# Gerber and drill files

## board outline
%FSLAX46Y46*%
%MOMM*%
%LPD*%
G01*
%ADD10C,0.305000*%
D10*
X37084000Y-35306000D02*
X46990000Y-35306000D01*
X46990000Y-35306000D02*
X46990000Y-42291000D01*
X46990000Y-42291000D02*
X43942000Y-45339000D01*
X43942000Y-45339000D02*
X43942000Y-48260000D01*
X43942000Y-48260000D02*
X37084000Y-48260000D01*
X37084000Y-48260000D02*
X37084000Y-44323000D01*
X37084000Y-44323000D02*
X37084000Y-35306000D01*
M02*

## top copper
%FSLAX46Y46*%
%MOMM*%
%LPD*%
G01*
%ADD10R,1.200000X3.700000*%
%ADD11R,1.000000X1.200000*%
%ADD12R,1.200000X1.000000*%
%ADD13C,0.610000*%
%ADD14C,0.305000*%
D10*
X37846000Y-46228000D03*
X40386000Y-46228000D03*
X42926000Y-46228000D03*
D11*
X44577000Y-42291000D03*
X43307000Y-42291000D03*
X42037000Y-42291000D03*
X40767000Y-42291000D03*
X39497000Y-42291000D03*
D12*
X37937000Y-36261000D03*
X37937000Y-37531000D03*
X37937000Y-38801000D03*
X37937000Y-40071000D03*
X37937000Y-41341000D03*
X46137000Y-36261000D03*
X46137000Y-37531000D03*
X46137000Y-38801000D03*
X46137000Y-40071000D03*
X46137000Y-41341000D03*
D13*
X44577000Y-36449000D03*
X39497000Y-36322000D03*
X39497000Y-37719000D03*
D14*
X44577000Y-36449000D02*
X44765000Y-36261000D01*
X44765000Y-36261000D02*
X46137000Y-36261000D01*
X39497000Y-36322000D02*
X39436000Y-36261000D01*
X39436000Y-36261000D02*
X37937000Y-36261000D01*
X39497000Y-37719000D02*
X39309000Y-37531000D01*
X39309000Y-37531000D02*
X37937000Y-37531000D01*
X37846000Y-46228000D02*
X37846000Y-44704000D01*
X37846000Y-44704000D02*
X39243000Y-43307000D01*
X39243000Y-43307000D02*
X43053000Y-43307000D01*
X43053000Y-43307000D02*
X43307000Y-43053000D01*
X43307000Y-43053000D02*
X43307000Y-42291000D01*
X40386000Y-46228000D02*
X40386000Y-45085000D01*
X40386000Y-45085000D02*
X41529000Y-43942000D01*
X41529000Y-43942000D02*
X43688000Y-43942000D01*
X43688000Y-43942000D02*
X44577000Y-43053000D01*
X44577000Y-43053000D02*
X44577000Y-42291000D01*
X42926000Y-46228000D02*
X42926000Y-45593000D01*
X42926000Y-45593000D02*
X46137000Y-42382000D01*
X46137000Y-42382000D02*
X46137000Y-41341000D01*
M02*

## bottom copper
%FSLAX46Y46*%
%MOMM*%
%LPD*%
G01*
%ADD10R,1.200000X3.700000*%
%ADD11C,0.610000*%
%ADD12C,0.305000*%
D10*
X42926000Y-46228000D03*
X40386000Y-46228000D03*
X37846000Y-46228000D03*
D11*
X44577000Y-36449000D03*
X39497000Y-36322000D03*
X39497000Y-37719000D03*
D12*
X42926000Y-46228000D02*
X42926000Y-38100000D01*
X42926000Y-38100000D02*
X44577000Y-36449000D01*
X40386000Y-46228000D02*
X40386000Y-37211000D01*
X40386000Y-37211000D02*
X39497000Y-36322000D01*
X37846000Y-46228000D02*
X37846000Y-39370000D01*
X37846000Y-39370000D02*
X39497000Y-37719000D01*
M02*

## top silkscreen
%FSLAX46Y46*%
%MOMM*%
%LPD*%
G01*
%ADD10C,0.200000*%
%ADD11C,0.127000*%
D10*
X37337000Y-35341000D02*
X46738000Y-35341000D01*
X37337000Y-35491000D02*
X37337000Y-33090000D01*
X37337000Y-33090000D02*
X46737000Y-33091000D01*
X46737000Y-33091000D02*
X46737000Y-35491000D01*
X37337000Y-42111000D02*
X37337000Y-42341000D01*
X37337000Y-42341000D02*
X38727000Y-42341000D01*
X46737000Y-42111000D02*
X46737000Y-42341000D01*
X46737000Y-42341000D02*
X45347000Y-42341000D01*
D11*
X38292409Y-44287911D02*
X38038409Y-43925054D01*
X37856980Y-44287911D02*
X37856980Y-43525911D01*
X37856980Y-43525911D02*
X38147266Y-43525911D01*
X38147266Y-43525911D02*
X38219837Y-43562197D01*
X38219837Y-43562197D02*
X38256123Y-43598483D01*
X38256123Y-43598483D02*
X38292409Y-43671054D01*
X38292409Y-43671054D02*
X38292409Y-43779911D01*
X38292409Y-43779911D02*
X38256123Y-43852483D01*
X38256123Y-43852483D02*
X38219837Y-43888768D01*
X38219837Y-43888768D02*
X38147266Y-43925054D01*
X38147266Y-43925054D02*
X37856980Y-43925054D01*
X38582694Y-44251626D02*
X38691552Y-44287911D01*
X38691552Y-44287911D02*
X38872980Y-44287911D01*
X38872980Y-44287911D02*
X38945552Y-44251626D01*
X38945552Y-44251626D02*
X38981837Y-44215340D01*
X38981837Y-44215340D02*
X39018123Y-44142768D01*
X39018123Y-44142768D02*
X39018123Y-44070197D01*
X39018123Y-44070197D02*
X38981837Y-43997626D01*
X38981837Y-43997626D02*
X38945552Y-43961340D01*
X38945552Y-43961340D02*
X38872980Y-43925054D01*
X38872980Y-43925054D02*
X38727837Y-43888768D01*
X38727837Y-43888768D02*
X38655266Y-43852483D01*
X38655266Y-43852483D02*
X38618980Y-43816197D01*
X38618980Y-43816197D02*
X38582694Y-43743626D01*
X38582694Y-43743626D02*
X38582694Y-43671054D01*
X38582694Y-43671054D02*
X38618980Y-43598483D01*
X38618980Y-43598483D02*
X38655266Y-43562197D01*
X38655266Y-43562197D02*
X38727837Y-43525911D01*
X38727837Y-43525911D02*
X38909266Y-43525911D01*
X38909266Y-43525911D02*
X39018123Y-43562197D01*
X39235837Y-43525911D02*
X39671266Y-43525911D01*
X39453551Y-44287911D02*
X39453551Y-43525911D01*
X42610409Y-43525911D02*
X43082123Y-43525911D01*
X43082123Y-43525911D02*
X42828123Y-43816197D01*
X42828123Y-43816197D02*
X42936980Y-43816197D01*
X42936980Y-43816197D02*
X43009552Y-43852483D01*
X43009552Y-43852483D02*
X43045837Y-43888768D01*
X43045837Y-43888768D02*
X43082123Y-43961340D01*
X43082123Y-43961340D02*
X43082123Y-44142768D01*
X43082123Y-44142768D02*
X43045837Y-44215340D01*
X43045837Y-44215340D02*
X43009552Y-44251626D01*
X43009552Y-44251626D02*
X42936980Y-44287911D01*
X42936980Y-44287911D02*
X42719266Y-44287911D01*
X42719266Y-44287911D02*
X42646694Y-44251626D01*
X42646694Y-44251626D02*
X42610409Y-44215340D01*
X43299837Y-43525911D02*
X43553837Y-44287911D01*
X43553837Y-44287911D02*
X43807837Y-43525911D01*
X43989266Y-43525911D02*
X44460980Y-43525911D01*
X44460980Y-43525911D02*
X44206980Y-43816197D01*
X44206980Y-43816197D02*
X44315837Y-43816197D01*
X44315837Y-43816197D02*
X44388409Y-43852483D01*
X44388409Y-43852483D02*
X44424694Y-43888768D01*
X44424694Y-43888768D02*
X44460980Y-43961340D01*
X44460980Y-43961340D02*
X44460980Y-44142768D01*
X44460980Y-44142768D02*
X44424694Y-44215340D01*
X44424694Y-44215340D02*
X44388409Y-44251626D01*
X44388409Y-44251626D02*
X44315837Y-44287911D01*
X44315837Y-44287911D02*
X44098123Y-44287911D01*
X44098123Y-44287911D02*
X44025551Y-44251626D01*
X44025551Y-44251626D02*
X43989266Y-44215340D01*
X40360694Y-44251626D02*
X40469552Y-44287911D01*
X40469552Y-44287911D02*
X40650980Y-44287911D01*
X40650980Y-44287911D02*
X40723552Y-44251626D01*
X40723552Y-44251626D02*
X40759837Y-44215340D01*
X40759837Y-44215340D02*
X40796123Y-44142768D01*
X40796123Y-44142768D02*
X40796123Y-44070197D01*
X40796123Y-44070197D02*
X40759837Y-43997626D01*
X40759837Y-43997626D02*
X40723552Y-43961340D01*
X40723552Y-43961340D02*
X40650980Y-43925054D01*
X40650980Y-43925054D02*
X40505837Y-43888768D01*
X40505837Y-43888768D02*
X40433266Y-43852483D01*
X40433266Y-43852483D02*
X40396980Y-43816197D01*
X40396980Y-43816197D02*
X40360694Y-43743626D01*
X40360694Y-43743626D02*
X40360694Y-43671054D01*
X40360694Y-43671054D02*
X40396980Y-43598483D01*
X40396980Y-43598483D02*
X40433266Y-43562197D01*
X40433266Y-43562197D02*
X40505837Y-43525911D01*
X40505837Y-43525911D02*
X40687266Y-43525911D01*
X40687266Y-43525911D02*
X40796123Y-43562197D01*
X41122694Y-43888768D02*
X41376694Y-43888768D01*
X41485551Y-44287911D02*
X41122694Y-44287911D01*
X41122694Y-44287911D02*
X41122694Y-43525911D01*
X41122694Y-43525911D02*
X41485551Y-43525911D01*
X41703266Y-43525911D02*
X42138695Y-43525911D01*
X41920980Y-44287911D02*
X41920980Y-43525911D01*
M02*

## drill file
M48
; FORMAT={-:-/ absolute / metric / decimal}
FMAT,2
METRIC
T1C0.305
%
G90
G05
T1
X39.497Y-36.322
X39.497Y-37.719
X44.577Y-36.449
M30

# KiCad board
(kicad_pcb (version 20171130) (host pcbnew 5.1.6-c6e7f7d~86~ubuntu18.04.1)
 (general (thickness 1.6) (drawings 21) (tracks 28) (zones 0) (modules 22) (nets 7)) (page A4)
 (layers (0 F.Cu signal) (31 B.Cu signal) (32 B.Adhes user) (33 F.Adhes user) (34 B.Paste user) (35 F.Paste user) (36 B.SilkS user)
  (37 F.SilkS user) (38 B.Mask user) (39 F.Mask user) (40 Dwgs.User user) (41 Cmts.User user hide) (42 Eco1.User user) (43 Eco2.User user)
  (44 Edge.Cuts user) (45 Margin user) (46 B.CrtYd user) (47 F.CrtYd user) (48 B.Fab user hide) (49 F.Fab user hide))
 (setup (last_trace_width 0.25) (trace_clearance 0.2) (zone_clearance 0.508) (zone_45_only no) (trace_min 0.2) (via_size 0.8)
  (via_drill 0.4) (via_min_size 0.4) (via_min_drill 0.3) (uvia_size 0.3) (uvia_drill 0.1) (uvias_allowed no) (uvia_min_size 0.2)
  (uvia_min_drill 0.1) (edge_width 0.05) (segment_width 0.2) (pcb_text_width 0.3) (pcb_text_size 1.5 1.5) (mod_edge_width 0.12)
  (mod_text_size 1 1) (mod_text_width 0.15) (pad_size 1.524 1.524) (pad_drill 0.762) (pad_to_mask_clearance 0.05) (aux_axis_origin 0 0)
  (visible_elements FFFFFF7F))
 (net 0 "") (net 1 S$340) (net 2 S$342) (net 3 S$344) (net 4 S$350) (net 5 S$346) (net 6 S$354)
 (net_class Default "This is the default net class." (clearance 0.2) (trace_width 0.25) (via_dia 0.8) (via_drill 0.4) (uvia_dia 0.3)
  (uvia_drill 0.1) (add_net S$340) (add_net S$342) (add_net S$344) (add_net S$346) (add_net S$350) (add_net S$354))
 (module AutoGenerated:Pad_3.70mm (layer F.Cu) (at 37.846 46.228)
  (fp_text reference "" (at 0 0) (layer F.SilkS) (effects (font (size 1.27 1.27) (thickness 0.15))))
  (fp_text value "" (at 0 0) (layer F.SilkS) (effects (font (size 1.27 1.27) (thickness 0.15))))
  (pad 1 smd rect (at 0 0 90) (size 3.7 1.2) (layers F.Cu F.Paste F.Mask) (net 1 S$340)))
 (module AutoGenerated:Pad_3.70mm (layer F.Cu) (at 40.386 46.228)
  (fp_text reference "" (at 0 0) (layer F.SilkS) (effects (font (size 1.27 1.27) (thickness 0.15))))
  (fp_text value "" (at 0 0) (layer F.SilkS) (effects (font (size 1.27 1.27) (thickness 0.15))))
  (pad 1 smd rect (at 0 0 90) (size 3.7 1.2) (layers F.Cu F.Paste F.Mask) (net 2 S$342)))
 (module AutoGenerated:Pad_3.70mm (layer F.Cu) (at 42.926 46.228)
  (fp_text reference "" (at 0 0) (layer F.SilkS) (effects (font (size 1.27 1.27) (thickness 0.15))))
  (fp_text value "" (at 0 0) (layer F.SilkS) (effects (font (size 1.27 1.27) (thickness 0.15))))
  (pad 1 smd rect (at 0 0 90) (size 3.7 1.2) (layers F.Cu F.Paste F.Mask) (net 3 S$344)))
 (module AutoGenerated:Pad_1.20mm (layer F.Cu) (at 44.577 42.291)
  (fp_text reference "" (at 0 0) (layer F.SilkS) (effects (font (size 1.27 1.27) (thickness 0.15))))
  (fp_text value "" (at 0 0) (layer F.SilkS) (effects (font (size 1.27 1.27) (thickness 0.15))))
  (pad 15 smd rect (at 0 0 270) (size 1.2 1) (layers F.Cu F.Paste F.Mask) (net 2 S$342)))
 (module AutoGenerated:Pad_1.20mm (layer F.Cu) (at 43.307 42.291)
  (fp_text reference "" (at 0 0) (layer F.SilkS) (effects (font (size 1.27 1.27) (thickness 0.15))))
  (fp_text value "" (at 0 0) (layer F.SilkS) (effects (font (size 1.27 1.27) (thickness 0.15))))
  (pad 14 smd rect (at 0 0 270) (size 1.2 1) (layers F.Cu F.Paste F.Mask) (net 1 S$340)))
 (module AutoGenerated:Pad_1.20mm (layer F.Cu) (at 42.037 42.291)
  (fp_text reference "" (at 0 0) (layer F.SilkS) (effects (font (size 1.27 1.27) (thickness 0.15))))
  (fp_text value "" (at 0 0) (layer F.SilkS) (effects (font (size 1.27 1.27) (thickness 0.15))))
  (pad 13 smd rect (at 0 0 270) (size 1.2 1) (layers F.Cu F.Paste F.Mask)))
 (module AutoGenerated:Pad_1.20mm (layer F.Cu) (at 40.767 42.291)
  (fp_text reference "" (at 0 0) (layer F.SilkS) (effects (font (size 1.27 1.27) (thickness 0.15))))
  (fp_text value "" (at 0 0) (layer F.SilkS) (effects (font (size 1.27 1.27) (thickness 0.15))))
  (pad 12 smd rect (at 0 0 270) (size 1.2 1) (layers F.Cu F.Paste F.Mask)))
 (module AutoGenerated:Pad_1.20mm (layer F.Cu) (at 39.497 42.291)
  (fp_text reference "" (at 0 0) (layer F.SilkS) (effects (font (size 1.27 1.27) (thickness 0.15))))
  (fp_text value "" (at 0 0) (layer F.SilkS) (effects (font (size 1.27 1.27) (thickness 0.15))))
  (pad 11 smd rect (at 0 0 270) (size 1.2 1) (layers F.Cu F.Paste F.Mask)))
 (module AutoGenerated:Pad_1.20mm (layer F.Cu) (at 37.937 36.261)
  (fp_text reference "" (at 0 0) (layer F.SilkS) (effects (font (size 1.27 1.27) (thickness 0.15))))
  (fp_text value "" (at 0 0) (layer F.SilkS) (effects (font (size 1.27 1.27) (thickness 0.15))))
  (pad 1 smd rect (at 0 0) (size 1.2 1) (layers F.Cu F.Paste F.Mask) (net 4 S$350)))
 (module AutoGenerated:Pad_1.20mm (layer F.Cu) (at 37.937 37.531)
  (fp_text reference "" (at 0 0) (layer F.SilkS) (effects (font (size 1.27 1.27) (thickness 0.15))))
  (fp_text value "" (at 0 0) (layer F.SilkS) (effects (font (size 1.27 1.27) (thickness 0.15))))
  (pad 2 smd rect (at 0 0) (size 1.2 1) (layers F.Cu F.Paste F.Mask) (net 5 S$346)))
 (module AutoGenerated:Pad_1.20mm (layer F.Cu) (at 37.937 38.801)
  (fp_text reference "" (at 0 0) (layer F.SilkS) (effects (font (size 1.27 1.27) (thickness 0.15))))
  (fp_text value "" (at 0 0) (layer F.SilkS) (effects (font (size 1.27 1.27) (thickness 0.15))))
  (pad 3 smd rect (at 0 0) (size 1.2 1) (layers F.Cu F.Paste F.Mask)))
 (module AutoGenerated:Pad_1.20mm (layer F.Cu) (at 37.937 40.071)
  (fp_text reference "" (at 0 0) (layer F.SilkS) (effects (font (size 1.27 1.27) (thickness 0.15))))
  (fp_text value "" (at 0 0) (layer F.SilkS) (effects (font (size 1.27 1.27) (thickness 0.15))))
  (pad 4 smd rect (at 0 0) (size 1.2 1) (layers F.Cu F.Paste F.Mask)))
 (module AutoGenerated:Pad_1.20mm (layer F.Cu) (at 37.937 41.341)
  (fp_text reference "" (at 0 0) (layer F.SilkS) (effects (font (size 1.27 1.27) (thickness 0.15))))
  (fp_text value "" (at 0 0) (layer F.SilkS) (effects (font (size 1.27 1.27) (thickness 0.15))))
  (pad 5 smd rect (at 0 0) (size 1.2 1) (layers F.Cu F.Paste F.Mask)))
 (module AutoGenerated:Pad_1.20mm (layer F.Cu) (at 46.137 36.261)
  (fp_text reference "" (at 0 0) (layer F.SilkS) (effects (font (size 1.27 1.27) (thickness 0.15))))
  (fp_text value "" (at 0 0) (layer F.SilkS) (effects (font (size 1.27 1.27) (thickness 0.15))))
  (pad 6 smd rect (at 0 0) (size 1.2 1) (layers F.Cu F.Paste F.Mask) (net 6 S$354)))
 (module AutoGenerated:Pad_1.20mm (layer F.Cu) (at 46.137 37.531)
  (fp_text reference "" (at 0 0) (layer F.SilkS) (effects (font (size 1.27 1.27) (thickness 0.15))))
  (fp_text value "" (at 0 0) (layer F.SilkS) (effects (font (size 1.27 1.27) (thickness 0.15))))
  (pad 7 smd rect (at 0 0) (size 1.2 1) (layers F.Cu F.Paste F.Mask)))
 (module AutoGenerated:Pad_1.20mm (layer F.Cu) (at 46.137 38.801)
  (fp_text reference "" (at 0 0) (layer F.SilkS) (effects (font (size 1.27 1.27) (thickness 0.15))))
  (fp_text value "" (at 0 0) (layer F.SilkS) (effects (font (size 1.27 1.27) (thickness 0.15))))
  (pad 8 smd rect (at 0 0) (size 1.2 1) (layers F.Cu F.Paste F.Mask)))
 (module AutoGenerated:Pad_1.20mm (layer F.Cu) (at 46.137 40.071)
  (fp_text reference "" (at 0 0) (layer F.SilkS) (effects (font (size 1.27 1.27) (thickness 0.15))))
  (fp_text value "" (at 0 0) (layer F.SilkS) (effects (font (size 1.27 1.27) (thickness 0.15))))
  (pad 9 smd rect (at 0 0) (size 1.2 1) (layers F.Cu F.Paste F.Mask)))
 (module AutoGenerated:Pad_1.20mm (layer F.Cu) (at 46.137 41.341)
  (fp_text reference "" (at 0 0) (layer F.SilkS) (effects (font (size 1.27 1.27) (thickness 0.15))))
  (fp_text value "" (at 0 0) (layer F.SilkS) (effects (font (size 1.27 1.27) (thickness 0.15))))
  (pad 10 smd rect (at 0 0) (size 1.2 1) (layers F.Cu F.Paste F.Mask) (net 3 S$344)))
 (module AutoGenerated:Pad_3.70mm (layer F.Cu) (at 42.926 46.228)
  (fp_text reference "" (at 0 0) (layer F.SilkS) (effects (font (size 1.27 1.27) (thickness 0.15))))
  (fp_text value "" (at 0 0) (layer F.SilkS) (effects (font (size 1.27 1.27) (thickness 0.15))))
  (pad 1 smd rect (at 0 0 90) (size 3.7 1.2) (layers B.Cu B.Paste B.Mask) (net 6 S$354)))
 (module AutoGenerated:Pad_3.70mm (layer F.Cu) (at 40.386 46.228)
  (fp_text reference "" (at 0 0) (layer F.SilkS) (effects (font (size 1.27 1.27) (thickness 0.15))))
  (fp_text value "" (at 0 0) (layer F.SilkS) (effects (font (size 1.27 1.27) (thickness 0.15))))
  (pad 1 smd rect (at 0 0 90) (size 3.7 1.2) (layers B.Cu B.Paste B.Mask) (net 4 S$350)))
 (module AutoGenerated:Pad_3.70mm (layer F.Cu) (at 37.846 46.228)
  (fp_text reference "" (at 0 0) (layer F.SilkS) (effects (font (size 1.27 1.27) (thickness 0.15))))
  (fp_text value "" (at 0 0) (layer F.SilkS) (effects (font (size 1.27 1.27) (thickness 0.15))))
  (pad 1 smd rect (at 0 0 90) (size 3.7 1.2) (layers B.Cu B.Paste B.Mask) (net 5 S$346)))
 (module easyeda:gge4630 (layer F.Cu) (at 42.037 37.719)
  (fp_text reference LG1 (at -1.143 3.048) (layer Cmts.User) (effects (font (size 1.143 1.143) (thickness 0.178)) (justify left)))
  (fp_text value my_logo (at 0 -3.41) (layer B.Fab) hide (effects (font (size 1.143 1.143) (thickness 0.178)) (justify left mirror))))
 (gr_line (start 37.084 35.306) (end 46.99 35.306) (layer Edge.Cuts) (width 0.305))
 (gr_line (start 46.99 35.306) (end 46.99 42.291) (layer Edge.Cuts) (width 0.305))
 (gr_line (start 46.99 42.291) (end 43.942 45.339) (layer Edge.Cuts) (width 0.305))
 (gr_line (start 43.942 45.339) (end 43.942 48.26) (layer Edge.Cuts) (width 0.305))
 (gr_line (start 43.942 48.26) (end 37.084 48.26) (layer Edge.Cuts) (width 0.305))
 (gr_line (start 37.084 48.26) (end 37.084 44.323) (layer Edge.Cuts) (width 0.305))
 (gr_line (start 37.084 44.323) (end 37.084 35.306) (layer Edge.Cuts) (width 0.305))
 (gr_line (start 37.337 35.341) (end 46.738 35.341) (layer F.SilkS) (width 0.2))
 (gr_line (start 37.337 35.491) (end 37.337 33.09) (layer F.SilkS) (width 0.2))
 (gr_line (start 37.337 33.09) (end 46.737 33.091) (layer F.SilkS) (width 0.2))
 (gr_line (start 46.737 33.091) (end 46.737 35.491) (layer F.SilkS) (width 0.2))
 (gr_line (start 37.337 42.111) (end 37.337 42.341) (layer F.SilkS) (width 0.2))
 (gr_line (start 37.337 42.341) (end 38.727 42.341) (layer F.SilkS) (width 0.2))
 (gr_line (start 46.737 42.111) (end 46.737 42.341) (layer F.SilkS) (width 0.2))
 (gr_line (start 46.737 42.341) (end 45.347 42.341) (layer F.SilkS) (width 0.2))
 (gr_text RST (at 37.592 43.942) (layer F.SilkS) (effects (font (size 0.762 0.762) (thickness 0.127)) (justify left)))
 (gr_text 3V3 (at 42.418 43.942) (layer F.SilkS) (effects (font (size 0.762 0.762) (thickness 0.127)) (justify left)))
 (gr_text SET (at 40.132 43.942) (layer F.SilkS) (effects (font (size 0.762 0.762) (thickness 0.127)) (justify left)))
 (segment (start 42.926 46.228) (end 42.926 38.1) (width 0.305) (layer B.Cu) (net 6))
 (segment (start 42.926 38.1) (end 44.577 36.449) (width 0.305) (layer B.Cu) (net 6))
 (segment (start 44.577 36.449) (end 44.765 36.261) (width 0.305) (layer F.Cu) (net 6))
 (segment (start 44.765 36.261) (end 46.137 36.261) (width 0.305) (layer F.Cu) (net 6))
 (via (at 44.577 36.449) (size 0.61) (drill 0.305) (layers F.Cu B.Cu) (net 6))
 (segment (start 40.386 46.228) (end 40.386 37.211) (width 0.305) (layer B.Cu) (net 4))
 (segment (start 40.386 37.211) (end 39.497 36.322) (width 0.305) (layer B.Cu) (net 4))
 (segment (start 39.497 36.322) (end 39.436 36.261) (width 0.305) (layer F.Cu) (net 4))
 (segment (start 39.436 36.261) (end 37.937 36.261) (width 0.305) (layer F.Cu) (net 4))
 (via (at 39.497 36.322) (size 0.61) (drill 0.305) (layers F.Cu B.Cu) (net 4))
 (segment (start 37.846 46.228) (end 37.846 39.37) (width 0.305) (layer B.Cu) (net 5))
 (segment (start 37.846 39.37) (end 39.497 37.719) (width 0.305) (layer B.Cu) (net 5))
 (segment (start 39.497 37.719) (end 39.309 37.531) (width 0.305) (layer F.Cu) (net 5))
 (segment (start 39.309 37.531) (end 37.937 37.531) (width 0.305) (layer F.Cu) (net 5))
 (via (at 39.497 37.719) (size 0.61) (drill 0.305) (layers F.Cu B.Cu) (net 5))
 (segment (start 37.846 46.228) (end 37.846 44.704) (width 0.305) (layer F.Cu) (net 1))
 (segment (start 37.846 44.704) (end 39.243 43.307) (width 0.305) (layer F.Cu) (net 1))
 (segment (start 39.243 43.307) (end 43.053 43.307) (width 0.305) (layer F.Cu) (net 1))
 (segment (start 43.053 43.307) (end 43.307 43.053) (width 0.305) (layer F.Cu) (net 1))
 (segment (start 43.307 43.053) (end 43.307 42.291) (width 0.305) (layer F.Cu) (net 1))
 (segment (start 40.386 46.228) (end 40.386 45.085) (width 0.305) (layer F.Cu) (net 2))
 (segment (start 40.386 45.085) (end 41.529 43.942) (width 0.305) (layer F.Cu) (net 2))
 (segment (start 41.529 43.942) (end 43.688 43.942) (width 0.305) (layer F.Cu) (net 2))
 (segment (start 43.688 43.942) (end 44.577 43.053) (width 0.305) (layer F.Cu) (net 2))
 (segment (start 44.577 43.053) (end 44.577 42.291) (width 0.305) (layer F.Cu) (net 2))
 (segment (start 42.926 46.228) (end 42.926 45.593) (width 0.305) (layer F.Cu) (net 3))
 (segment (start 42.926 45.593) (end 46.137 42.382) (width 0.305) (layer F.Cu) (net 3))
 (segment (start 46.137 42.382) (end 46.137 41.341) (width 0.305) (layer F.Cu) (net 3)))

